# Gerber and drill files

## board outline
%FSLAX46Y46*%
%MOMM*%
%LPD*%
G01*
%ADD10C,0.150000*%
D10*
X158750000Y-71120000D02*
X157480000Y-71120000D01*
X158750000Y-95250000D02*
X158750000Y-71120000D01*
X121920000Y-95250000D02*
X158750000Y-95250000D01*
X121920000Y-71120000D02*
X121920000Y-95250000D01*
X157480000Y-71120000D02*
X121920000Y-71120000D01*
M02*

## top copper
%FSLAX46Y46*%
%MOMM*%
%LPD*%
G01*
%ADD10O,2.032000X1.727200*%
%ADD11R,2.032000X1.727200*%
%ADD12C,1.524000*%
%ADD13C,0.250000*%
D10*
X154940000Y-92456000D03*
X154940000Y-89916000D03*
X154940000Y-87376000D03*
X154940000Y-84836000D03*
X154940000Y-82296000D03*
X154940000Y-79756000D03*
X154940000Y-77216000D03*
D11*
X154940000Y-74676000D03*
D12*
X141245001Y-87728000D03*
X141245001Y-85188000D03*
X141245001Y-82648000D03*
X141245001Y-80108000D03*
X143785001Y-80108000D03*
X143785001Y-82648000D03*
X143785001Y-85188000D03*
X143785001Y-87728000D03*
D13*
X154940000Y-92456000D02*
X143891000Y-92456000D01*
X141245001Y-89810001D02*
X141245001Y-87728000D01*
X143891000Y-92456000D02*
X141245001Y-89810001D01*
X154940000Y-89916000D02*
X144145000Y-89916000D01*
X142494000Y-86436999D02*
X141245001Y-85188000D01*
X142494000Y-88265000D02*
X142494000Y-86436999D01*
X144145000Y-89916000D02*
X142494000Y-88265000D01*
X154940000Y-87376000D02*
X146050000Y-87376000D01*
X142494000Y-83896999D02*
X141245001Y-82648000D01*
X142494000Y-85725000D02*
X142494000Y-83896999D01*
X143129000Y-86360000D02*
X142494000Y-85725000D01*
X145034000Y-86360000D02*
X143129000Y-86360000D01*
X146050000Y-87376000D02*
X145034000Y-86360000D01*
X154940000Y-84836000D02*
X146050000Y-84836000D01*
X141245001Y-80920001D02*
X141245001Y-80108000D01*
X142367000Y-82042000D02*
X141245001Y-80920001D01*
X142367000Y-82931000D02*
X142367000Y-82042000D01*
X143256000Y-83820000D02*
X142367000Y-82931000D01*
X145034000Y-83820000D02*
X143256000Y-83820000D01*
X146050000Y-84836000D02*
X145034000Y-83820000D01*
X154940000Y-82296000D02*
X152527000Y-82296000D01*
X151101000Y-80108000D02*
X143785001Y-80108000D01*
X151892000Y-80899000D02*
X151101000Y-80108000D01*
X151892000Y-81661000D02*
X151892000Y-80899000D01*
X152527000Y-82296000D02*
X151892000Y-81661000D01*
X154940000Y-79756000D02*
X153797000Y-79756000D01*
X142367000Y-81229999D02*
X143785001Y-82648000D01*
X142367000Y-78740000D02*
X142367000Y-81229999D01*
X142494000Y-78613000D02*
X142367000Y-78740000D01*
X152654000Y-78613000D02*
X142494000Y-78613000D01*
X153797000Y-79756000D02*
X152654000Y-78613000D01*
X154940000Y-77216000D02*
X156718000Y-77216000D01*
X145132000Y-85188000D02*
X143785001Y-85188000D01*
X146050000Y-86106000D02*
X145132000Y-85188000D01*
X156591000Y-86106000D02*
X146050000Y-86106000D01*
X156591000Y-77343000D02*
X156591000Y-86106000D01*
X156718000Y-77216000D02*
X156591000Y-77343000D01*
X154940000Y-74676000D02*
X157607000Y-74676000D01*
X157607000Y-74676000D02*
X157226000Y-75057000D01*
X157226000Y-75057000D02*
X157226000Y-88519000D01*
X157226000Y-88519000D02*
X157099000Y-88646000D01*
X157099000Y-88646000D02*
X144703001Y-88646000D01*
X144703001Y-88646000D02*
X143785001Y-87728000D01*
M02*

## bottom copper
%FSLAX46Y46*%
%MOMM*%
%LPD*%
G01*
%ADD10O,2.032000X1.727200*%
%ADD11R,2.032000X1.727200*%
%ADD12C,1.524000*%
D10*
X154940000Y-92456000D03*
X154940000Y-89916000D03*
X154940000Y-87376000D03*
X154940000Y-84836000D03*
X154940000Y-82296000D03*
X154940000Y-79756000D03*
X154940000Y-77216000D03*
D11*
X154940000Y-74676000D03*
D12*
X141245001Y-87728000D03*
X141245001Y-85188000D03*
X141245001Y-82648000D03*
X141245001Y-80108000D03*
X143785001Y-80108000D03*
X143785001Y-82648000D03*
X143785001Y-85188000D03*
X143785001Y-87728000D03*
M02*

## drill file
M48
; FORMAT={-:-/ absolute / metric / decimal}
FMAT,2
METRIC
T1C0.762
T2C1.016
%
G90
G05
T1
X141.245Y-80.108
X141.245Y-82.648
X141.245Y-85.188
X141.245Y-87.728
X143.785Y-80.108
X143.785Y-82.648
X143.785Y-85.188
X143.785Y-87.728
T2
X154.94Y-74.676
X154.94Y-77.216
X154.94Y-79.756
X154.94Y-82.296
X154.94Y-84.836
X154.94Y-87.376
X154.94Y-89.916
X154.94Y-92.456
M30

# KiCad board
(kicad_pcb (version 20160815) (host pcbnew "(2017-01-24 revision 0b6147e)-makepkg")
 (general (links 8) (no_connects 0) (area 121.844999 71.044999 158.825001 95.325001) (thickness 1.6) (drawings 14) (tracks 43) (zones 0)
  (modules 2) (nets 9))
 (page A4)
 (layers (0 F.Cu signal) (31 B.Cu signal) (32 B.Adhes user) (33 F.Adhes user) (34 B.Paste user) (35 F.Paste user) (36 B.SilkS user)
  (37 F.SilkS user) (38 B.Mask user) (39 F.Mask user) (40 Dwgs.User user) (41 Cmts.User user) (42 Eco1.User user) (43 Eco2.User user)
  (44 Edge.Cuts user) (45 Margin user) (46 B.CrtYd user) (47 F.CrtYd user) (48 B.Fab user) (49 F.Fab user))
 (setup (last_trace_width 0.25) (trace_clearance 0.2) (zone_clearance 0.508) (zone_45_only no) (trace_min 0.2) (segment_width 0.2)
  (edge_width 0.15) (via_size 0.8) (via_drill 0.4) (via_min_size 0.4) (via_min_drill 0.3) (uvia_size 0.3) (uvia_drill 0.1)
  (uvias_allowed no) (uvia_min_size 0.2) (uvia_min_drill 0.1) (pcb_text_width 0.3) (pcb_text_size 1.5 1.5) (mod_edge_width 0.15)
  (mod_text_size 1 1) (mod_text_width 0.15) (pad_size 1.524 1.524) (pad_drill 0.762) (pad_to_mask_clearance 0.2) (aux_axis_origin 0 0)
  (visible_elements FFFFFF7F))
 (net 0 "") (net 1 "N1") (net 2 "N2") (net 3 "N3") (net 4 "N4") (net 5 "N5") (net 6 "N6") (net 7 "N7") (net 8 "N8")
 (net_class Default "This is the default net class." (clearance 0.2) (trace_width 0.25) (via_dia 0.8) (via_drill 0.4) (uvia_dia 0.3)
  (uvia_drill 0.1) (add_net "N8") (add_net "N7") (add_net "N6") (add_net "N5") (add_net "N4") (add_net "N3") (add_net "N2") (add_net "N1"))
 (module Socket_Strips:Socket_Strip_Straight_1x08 (layer F.Cu) (at 154.94 74.676 270)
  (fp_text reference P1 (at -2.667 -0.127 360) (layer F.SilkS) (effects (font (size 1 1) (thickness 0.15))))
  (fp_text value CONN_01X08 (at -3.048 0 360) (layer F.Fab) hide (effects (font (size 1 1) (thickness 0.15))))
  (pad 8 thru_hole oval (at 17.78 0 270) (size 1.7272 2.032) (drill 1.016) (layers *.Cu *.Mask) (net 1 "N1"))
  (pad 7 thru_hole oval (at 15.24 0 270) (size 1.7272 2.032) (drill 1.016) (layers *.Cu *.Mask) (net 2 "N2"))
  (pad 6 thru_hole oval (at 12.7 0 270) (size 1.7272 2.032) (drill 1.016) (layers *.Cu *.Mask) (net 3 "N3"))
  (pad 5 thru_hole oval (at 10.16 0 270) (size 1.7272 2.032) (drill 1.016) (layers *.Cu *.Mask) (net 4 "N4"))
  (pad 4 thru_hole oval (at 7.62 0 270) (size 1.7272 2.032) (drill 1.016) (layers *.Cu *.Mask) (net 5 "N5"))
  (pad 3 thru_hole oval (at 5.08 0 270) (size 1.7272 2.032) (drill 1.016) (layers *.Cu *.Mask) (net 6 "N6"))
  (pad 2 thru_hole oval (at 2.54 0 270) (size 1.7272 2.032) (drill 1.016) (layers *.Cu *.Mask) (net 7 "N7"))
  (pad 1 thru_hole rect (at 0 0 270) (size 1.7272 2.032) (drill 1.016) (layers *.Cu *.Mask) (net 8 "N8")))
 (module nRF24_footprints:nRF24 (layer F.Cu) (at 133.625001 77.568)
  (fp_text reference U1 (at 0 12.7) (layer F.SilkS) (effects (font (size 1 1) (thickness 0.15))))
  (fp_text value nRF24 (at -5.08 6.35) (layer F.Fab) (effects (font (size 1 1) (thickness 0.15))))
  (pad 7 thru_hole circle (at 7.62 10.16) (size 1.524 1.524) (drill 0.762) (layers *.Cu *.Mask) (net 1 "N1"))
  (pad 6 thru_hole circle (at 7.62 7.62) (size 1.524 1.524) (drill 0.762) (layers *.Cu *.Mask) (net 2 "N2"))
  (pad 5 thru_hole circle (at 7.62 5.08) (size 1.524 1.524) (drill 0.762) (layers *.Cu *.Mask) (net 3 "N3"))
  (pad 4 thru_hole circle (at 7.62 2.54) (size 1.524 1.524) (drill 0.762) (layers *.Cu *.Mask) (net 4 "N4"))
  (pad 3 thru_hole circle (at 10.16 2.54) (size 1.524 1.524) (drill 0.762) (layers *.Cu *.Mask) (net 5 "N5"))
  (pad 2 thru_hole circle (at 10.16 5.08) (size 1.524 1.524) (drill 0.762) (layers *.Cu *.Mask) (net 6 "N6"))
  (pad 1 thru_hole circle (at 10.16 7.62) (size 1.524 1.524) (drill 0.762) (layers *.Cu *.Mask) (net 7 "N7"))
  (pad 0 thru_hole circle (at 10.16 10.16) (size 1.524 1.524) (drill 0.762) (layers *.Cu *.Mask) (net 8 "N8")))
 (gr_line (start 158.75 71.12) (end 157.48 71.12) (angle 90) (layer Edge.Cuts) (width 0.15))
 (gr_line (start 158.75 95.25) (end 158.75 71.12) (angle 90) (layer Edge.Cuts) (width 0.15))
 (gr_line (start 121.92 95.25) (end 158.75 95.25) (angle 90) (layer Edge.Cuts) (width 0.15))
 (gr_line (start 121.92 71.12) (end 121.92 95.25) (angle 90) (layer Edge.Cuts) (width 0.15))
 (gr_line (start 157.48 71.12) (end 121.92 71.12) (angle 90) (layer Edge.Cuts) (width 0.15))
 (segment (start 154.94 92.456) (end 143.891 92.456) (width 0.25) (layer F.Cu) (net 1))
 (segment (start 141.245001 89.810001) (end 141.245001 87.728) (width 0.25) (layer F.Cu) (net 1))
 (segment (start 143.891 92.456) (end 141.245001 89.810001) (width 0.25) (layer F.Cu) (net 1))
 (segment (start 154.94 89.916) (end 144.145 89.916) (width 0.25) (layer F.Cu) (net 2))
 (segment (start 142.494 86.436999) (end 141.245001 85.188) (width 0.25) (layer F.Cu) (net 2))
 (segment (start 142.494 88.265) (end 142.494 86.436999) (width 0.25) (layer F.Cu) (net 2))
 (segment (start 144.145 89.916) (end 142.494 88.265) (width 0.25) (layer F.Cu) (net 2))
 (segment (start 154.94 87.376) (end 146.05 87.376) (width 0.25) (layer F.Cu) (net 3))
 (segment (start 142.494 83.896999) (end 141.245001 82.648) (width 0.25) (layer F.Cu) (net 3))
 (segment (start 142.494 85.725) (end 142.494 83.896999) (width 0.25) (layer F.Cu) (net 3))
 (segment (start 143.129 86.36) (end 142.494 85.725) (width 0.25) (layer F.Cu) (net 3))
 (segment (start 145.034 86.36) (end 143.129 86.36) (width 0.25) (layer F.Cu) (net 3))
 (segment (start 146.05 87.376) (end 145.034 86.36) (width 0.25) (layer F.Cu) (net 3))
 (segment (start 154.94 84.836) (end 146.05 84.836) (width 0.25) (layer F.Cu) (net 4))
 (segment (start 141.245001 80.920001) (end 141.245001 80.108) (width 0.25) (layer F.Cu) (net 4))
 (segment (start 142.367 82.042) (end 141.245001 80.920001) (width 0.25) (layer F.Cu) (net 4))
 (segment (start 142.367 82.931) (end 142.367 82.042) (width 0.25) (layer F.Cu) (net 4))
 (segment (start 143.256 83.82) (end 142.367 82.931) (width 0.25) (layer F.Cu) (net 4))
 (segment (start 145.034 83.82) (end 143.256 83.82) (width 0.25) (layer F.Cu) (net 4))
 (segment (start 146.05 84.836) (end 145.034 83.82) (width 0.25) (layer F.Cu) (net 4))
 (segment (start 154.94 82.296) (end 152.527 82.296) (width 0.25) (layer F.Cu) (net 5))
 (segment (start 151.101 80.108) (end 143.785001 80.108) (width 0.25) (layer F.Cu) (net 5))
 (segment (start 151.892 80.899) (end 151.101 80.108) (width 0.25) (layer F.Cu) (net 5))
 (segment (start 151.892 81.661) (end 151.892 80.899) (width 0.25) (layer F.Cu) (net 5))
 (segment (start 152.527 82.296) (end 151.892 81.661) (width 0.25) (layer F.Cu) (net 5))
 (segment (start 154.94 79.756) (end 153.797 79.756) (width 0.25) (layer F.Cu) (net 6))
 (segment (start 142.367 81.229999) (end 143.785001 82.648) (width 0.25) (layer F.Cu) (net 6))
 (segment (start 142.367 78.74) (end 142.367 81.229999) (width 0.25) (layer F.Cu) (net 6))
 (segment (start 142.494 78.613) (end 142.367 78.74) (width 0.25) (layer F.Cu) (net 6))
 (segment (start 152.654 78.613) (end 142.494 78.613) (width 0.25) (layer F.Cu) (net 6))
 (segment (start 153.797 79.756) (end 152.654 78.613) (width 0.25) (layer F.Cu) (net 6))
 (segment (start 154.94 77.216) (end 156.718 77.216) (width 0.25) (layer F.Cu) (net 7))
 (segment (start 145.132 85.188) (end 143.785001 85.188) (width 0.25) (layer F.Cu) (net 7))
 (segment (start 146.05 86.106) (end 145.132 85.188) (width 0.25) (layer F.Cu) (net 7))
 (segment (start 156.591 86.106) (end 146.05 86.106) (width 0.25) (layer F.Cu) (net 7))
 (segment (start 156.591 77.343) (end 156.591 86.106) (width 0.25) (layer F.Cu) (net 7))
 (segment (start 156.718 77.216) (end 156.591 77.343) (width 0.25) (layer F.Cu) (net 7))
 (segment (start 154.94 74.676) (end 157.607 74.676) (width 0.25) (layer F.Cu) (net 8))
 (segment (start 157.607 74.676) (end 157.226 75.057) (width 0.25) (layer F.Cu) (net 8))
 (segment (start 157.226 75.057) (end 157.226 88.519) (width 0.25) (layer F.Cu) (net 8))
 (segment (start 157.226 88.519) (end 157.099 88.646) (width 0.25) (layer F.Cu) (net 8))
 (segment (start 157.099 88.646) (end 144.703001 88.646) (width 0.25) (layer F.Cu) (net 8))
 (segment (start 144.703001 88.646) (end 143.785001 87.728) (width 0.25) (layer F.Cu) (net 8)))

